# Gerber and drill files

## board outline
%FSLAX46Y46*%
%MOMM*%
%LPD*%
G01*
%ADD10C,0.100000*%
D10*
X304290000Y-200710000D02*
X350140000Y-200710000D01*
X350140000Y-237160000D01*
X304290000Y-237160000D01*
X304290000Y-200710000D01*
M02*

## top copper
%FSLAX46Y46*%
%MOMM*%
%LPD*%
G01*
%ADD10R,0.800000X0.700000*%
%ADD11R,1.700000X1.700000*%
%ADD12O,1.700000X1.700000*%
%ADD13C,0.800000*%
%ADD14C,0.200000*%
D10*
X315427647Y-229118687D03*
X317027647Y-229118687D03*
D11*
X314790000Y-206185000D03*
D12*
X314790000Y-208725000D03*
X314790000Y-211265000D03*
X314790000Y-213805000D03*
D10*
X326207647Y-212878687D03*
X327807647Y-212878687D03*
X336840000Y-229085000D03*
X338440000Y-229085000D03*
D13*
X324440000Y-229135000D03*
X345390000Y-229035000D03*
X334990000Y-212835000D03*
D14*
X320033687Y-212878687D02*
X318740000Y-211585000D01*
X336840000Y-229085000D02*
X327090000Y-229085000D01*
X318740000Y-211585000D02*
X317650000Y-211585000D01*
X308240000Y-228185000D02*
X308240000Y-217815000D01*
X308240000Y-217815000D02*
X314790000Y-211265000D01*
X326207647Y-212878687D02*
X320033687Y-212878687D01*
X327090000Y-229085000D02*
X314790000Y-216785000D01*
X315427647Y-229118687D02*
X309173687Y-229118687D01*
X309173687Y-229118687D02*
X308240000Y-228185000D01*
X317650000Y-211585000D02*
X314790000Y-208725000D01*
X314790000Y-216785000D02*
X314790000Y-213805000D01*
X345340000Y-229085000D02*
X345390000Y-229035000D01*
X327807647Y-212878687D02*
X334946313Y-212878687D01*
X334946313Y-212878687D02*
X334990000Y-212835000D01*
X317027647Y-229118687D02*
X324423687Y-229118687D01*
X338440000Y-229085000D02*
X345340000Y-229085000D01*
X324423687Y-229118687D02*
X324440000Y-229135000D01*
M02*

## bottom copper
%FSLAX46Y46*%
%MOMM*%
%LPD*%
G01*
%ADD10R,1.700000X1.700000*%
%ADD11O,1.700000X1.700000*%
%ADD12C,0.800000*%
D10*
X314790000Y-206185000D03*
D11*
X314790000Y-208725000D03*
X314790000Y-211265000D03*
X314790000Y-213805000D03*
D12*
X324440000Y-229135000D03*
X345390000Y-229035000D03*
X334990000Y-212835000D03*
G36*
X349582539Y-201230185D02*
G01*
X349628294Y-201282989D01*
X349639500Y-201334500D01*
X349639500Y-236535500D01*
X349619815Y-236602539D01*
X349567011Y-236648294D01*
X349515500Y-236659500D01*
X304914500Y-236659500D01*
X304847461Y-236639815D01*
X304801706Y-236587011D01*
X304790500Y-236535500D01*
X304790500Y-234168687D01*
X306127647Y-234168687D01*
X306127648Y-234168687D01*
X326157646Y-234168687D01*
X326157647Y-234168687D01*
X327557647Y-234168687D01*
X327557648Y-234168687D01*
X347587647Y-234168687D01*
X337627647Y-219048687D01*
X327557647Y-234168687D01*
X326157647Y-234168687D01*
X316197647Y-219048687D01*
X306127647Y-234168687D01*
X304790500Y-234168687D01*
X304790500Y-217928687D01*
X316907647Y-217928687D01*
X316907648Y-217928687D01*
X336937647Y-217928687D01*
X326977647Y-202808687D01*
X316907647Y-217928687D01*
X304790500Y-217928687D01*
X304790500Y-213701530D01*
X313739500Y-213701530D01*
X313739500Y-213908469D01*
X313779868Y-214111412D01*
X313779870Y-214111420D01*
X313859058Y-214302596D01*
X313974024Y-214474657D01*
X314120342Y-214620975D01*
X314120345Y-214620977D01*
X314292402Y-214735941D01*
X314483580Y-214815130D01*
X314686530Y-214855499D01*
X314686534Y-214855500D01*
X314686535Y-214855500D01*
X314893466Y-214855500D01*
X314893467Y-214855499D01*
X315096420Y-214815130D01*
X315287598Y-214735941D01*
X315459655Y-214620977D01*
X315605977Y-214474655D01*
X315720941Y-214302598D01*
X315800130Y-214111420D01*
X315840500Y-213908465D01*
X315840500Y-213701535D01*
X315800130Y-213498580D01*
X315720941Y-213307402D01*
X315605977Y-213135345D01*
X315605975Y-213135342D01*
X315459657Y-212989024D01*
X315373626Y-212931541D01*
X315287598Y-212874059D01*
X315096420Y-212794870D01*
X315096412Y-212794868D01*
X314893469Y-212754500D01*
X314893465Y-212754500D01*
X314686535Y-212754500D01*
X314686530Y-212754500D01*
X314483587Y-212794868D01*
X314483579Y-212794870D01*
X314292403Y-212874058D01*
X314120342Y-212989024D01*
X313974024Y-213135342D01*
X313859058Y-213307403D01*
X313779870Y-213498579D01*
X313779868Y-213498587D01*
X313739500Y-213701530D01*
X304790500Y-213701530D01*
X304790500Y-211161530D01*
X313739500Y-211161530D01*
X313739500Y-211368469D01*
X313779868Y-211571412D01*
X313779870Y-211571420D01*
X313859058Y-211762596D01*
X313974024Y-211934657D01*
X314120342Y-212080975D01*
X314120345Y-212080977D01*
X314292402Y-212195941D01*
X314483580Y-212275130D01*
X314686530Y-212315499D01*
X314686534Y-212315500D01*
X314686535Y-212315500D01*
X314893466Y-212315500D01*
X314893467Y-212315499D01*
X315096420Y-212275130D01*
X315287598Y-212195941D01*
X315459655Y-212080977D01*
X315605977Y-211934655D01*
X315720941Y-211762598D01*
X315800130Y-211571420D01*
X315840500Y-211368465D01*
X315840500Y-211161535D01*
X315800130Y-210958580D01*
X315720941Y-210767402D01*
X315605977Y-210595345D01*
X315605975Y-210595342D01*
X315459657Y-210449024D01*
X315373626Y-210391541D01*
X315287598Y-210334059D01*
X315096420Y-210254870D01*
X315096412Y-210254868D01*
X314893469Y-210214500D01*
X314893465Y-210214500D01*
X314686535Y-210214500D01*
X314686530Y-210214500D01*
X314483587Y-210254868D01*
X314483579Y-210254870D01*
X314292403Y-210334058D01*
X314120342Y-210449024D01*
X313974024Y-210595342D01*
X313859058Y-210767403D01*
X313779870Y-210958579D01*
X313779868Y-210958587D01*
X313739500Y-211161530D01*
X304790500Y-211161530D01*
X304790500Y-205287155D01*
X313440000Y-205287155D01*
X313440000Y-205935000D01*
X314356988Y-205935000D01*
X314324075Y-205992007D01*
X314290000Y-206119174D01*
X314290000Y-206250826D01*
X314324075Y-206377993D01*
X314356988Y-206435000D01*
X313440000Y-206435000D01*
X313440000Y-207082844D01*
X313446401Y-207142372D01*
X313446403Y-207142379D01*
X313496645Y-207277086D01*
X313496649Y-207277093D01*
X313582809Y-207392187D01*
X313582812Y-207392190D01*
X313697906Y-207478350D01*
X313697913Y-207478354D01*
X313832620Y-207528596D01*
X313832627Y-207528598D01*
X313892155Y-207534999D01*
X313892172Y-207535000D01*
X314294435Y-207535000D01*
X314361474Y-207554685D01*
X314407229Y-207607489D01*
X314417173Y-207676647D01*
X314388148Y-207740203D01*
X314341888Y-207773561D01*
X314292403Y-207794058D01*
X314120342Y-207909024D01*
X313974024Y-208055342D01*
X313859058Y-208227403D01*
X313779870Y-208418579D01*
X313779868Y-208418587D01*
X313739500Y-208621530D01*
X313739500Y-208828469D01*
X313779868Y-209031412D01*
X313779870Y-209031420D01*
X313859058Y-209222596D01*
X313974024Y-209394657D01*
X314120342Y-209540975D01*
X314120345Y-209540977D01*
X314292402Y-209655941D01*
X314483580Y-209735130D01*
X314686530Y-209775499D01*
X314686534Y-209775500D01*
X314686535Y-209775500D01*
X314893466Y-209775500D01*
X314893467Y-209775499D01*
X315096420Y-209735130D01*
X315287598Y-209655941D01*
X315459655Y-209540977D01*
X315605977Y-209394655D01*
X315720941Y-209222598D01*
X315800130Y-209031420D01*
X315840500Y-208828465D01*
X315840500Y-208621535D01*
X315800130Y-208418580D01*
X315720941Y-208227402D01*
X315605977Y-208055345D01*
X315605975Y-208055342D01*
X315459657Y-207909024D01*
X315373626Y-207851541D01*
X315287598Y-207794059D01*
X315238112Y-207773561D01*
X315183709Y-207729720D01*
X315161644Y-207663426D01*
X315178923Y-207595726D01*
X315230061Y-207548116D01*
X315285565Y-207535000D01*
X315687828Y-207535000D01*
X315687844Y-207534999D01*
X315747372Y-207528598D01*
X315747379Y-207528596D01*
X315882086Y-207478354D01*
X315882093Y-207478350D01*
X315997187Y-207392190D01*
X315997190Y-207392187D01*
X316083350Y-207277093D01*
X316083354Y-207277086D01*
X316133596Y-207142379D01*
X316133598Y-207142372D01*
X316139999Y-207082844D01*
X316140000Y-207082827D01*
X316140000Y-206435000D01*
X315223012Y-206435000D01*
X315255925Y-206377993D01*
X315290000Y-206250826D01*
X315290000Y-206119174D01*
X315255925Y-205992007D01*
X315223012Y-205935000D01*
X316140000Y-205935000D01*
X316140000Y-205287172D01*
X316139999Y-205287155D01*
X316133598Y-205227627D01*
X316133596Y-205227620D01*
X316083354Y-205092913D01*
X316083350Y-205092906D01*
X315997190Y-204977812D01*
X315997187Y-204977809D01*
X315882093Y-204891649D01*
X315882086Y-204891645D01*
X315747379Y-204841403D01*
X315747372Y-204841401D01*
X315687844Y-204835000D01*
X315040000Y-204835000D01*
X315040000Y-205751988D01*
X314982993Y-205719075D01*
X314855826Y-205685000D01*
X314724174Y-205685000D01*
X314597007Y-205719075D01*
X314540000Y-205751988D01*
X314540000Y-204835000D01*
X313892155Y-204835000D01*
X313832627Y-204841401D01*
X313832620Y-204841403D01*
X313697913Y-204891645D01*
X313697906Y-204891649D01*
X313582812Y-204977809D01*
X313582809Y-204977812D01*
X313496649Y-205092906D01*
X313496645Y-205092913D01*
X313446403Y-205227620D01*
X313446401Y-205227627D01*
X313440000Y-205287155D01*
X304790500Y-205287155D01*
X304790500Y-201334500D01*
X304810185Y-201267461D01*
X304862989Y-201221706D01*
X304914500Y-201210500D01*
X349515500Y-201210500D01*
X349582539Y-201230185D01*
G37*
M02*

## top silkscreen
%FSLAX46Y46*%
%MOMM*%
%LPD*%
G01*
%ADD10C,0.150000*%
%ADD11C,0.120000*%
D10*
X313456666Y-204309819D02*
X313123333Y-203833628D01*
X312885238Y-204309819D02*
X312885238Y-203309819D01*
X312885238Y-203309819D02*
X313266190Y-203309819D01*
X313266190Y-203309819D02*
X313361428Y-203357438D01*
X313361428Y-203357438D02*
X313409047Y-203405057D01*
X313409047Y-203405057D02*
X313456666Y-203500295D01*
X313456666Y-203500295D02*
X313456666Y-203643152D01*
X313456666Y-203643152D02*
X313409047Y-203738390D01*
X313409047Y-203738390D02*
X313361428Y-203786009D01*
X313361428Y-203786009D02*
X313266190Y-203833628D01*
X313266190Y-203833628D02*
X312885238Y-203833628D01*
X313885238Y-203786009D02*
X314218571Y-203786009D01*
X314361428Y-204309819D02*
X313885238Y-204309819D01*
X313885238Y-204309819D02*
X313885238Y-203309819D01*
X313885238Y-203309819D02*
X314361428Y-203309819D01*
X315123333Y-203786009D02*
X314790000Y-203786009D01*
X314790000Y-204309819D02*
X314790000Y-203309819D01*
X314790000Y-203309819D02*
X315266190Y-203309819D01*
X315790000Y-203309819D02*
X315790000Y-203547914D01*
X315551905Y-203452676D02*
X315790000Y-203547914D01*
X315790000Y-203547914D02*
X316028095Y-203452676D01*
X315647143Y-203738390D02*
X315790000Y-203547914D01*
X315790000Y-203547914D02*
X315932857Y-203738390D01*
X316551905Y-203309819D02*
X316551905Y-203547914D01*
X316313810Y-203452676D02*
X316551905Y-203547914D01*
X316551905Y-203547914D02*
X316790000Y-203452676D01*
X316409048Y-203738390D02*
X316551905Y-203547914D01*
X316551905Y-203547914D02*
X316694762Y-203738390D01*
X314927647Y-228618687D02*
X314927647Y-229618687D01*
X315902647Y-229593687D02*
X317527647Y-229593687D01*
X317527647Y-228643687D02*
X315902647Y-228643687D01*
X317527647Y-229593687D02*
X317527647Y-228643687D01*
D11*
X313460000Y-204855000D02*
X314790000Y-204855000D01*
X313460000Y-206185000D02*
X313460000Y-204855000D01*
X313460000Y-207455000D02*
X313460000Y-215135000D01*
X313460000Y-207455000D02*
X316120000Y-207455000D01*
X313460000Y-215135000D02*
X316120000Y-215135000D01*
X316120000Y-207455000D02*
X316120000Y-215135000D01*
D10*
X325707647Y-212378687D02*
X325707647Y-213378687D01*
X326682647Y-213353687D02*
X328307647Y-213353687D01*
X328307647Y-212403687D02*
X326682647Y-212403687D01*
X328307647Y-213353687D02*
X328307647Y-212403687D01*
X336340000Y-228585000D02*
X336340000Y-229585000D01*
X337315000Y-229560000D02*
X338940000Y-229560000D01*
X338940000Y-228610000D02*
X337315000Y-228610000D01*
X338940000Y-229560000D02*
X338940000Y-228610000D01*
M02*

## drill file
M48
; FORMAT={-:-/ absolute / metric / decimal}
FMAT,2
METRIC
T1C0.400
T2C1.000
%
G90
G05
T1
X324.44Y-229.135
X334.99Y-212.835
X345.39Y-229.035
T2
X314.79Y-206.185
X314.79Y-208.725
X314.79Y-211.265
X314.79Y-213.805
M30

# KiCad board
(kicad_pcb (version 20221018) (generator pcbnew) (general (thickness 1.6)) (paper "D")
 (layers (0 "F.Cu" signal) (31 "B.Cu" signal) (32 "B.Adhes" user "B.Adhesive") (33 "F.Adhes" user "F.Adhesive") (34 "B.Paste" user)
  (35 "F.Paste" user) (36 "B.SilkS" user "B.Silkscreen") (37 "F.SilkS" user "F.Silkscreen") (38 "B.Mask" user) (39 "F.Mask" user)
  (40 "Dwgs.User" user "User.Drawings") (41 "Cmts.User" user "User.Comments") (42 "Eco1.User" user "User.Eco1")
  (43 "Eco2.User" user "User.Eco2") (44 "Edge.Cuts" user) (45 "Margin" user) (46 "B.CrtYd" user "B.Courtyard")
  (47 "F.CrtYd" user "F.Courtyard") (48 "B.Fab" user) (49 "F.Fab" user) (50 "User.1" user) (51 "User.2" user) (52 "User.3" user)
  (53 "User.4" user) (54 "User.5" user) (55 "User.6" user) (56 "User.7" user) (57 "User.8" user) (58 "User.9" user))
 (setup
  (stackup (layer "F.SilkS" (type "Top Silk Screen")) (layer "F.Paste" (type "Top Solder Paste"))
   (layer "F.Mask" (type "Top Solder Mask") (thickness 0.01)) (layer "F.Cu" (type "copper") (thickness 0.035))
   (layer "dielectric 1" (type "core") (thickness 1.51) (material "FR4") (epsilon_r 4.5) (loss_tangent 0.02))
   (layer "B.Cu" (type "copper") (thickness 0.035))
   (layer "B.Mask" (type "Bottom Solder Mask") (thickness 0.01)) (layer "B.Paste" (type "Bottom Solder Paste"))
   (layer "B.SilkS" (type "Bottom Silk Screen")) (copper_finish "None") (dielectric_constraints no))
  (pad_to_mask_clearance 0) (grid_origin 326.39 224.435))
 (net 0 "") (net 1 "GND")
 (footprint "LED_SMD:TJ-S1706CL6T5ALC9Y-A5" (layer "F.Cu") (at 315.427647 229.118687)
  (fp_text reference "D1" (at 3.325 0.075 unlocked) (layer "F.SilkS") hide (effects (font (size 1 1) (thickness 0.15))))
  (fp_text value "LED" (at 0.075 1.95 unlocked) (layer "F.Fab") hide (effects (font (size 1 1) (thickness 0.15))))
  (fp_line (start -0.5 -0.5) (end -0.5 0.5) (stroke (width 0.15) (type default)) (layer "F.SilkS"))
  (fp_line (start 0.475 0.475) (end 2.1 0.475) (stroke (width 0.15) (type default)) (layer "F.SilkS"))
  (fp_line (start 2.1 -0.475) (end 0.475 -0.475) (stroke (width 0.15) (type default)) (layer "F.SilkS"))
  (fp_line (start 2.1 0.475) (end 2.1 -0.475) (stroke (width 0.15) (type default)) (layer "F.SilkS"))
  (pad "1" smd rect (at 0 0) (size 0.8 0.7) (layers "F.Cu" "F.Paste" "F.Mask") (thermal_bridge_angle 45))
  (pad "2" smd rect (at 1.6 0) (size 0.8 0.7) (layers "F.Cu" "F.Paste" "F.Mask") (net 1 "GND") (thermal_bridge_angle 45)))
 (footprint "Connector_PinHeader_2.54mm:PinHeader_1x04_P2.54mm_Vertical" (layer "F.Cu") (at 314.79 206.185)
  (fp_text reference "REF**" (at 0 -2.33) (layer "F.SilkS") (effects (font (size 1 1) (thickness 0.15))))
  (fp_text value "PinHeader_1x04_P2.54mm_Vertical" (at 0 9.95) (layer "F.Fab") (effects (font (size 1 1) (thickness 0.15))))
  (fp_line (start -1.33 -1.33) (end 0 -1.33) (stroke (width 0.12) (type solid)) (layer "F.SilkS"))
  (fp_line (start -1.33 0) (end -1.33 -1.33) (stroke (width 0.12) (type solid)) (layer "F.SilkS"))
  (fp_line (start -1.33 1.27) (end -1.33 8.95) (stroke (width 0.12) (type solid)) (layer "F.SilkS"))
  (fp_line (start -1.33 1.27) (end 1.33 1.27) (stroke (width 0.12) (type solid)) (layer "F.SilkS"))
  (fp_line (start -1.33 8.95) (end 1.33 8.95) (stroke (width 0.12) (type solid)) (layer "F.SilkS"))
  (fp_line (start 1.33 1.27) (end 1.33 8.95) (stroke (width 0.12) (type solid)) (layer "F.SilkS"))
  (pad "1" thru_hole rect (at 0 0) (size 1.7 1.7) (drill 1) (layers "*.Cu" "*.Mask") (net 1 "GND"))
  (pad "2" thru_hole oval (at 0 2.54) (size 1.7 1.7) (drill 1) (layers "*.Cu" "*.Mask"))
  (pad "3" thru_hole oval (at 0 5.08) (size 1.7 1.7) (drill 1) (layers "*.Cu" "*.Mask"))
  (pad "4" thru_hole oval (at 0 7.62) (size 1.7 1.7) (drill 1) (layers "*.Cu" "*.Mask")))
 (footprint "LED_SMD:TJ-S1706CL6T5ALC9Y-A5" (layer "F.Cu") (at 326.207647 212.878687)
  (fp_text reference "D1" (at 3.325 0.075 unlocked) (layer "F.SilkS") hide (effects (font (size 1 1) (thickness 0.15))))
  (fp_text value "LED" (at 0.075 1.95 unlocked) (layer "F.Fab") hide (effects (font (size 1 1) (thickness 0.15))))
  (fp_line (start -0.5 -0.5) (end -0.5 0.5) (stroke (width 0.15) (type default)) (layer "F.SilkS"))
  (fp_line (start 0.475 0.475) (end 2.1 0.475) (stroke (width 0.15) (type default)) (layer "F.SilkS"))
  (fp_line (start 2.1 -0.475) (end 0.475 -0.475) (stroke (width 0.15) (type default)) (layer "F.SilkS"))
  (fp_line (start 2.1 0.475) (end 2.1 -0.475) (stroke (width 0.15) (type default)) (layer "F.SilkS"))
  (pad "1" smd rect (at 0 0) (size 0.8 0.7) (layers "F.Cu" "F.Paste" "F.Mask") (thermal_bridge_angle 45))
  (pad "2" smd rect (at 1.6 0) (size 0.8 0.7) (layers "F.Cu" "F.Paste" "F.Mask") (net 1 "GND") (thermal_bridge_angle 45)))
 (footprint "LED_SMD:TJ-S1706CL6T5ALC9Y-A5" (layer "F.Cu") (at 336.84 229.085)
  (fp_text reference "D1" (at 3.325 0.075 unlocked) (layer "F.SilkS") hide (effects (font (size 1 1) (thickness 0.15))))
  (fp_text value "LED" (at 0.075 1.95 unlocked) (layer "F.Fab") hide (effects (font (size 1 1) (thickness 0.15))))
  (fp_line (start -0.5 -0.5) (end -0.5 0.5) (stroke (width 0.15) (type default)) (layer "F.SilkS"))
  (fp_line (start 0.475 0.475) (end 2.1 0.475) (stroke (width 0.15) (type default)) (layer "F.SilkS"))
  (fp_line (start 2.1 -0.475) (end 0.475 -0.475) (stroke (width 0.15) (type default)) (layer "F.SilkS"))
  (fp_line (start 2.1 0.475) (end 2.1 -0.475) (stroke (width 0.15) (type default)) (layer "F.SilkS"))
  (pad "1" smd rect (at 0 0) (size 0.8 0.7) (layers "F.Cu" "F.Paste" "F.Mask") (thermal_bridge_angle 45))
  (pad "2" smd rect (at 1.6 0) (size 0.8 0.7) (layers "F.Cu" "F.Paste" "F.Mask") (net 1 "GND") (thermal_bridge_angle 45)))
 (gr_rect (start 304.29 200.71) (end 350.14 237.16) (stroke (width 0.1) (type default)) (fill none) (layer "Edge.Cuts"))
 (segment (start 320.033687 212.878687) (end 318.74 211.585) (width 0.2) (layer "F.Cu") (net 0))
 (segment (start 336.84 229.085) (end 327.09 229.085) (width 0.2) (layer "F.Cu") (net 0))
 (segment (start 318.74 211.585) (end 317.65 211.585) (width 0.2) (layer "F.Cu") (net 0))
 (segment (start 308.24 228.185) (end 308.24 217.815) (width 0.2) (layer "F.Cu") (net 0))
 (segment (start 308.24 217.815) (end 314.79 211.265) (width 0.2) (layer "F.Cu") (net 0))
 (segment (start 326.207647 212.878687) (end 320.033687 212.878687) (width 0.2) (layer "F.Cu") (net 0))
 (segment (start 327.09 229.085) (end 314.79 216.785) (width 0.2) (layer "F.Cu") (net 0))
 (segment (start 315.427647 229.118687) (end 309.173687 229.118687) (width 0.2) (layer "F.Cu") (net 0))
 (segment (start 309.173687 229.118687) (end 308.24 228.185) (width 0.2) (layer "F.Cu") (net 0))
 (segment (start 317.65 211.585) (end 314.79 208.725) (width 0.2) (layer "F.Cu") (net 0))
 (segment (start 314.79 216.785) (end 314.79 213.805) (width 0.2) (layer "F.Cu") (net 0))
 (segment (start 345.34 229.085) (end 345.39 229.035) (width 0.2) (layer "F.Cu") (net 1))
 (segment (start 327.807647 212.878687) (end 334.946313 212.878687) (width 0.2) (layer "F.Cu") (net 1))
 (segment (start 334.946313 212.878687) (end 334.99 212.835) (width 0.2) (layer "F.Cu") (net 1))
 (segment (start 317.027647 229.118687) (end 324.423687 229.118687) (width 0.2) (layer "F.Cu") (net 1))
 (segment (start 338.44 229.085) (end 345.34 229.085) (width 0.2) (layer "F.Cu") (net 1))
 (segment (start 324.423687 229.118687) (end 324.44 229.135) (width 0.2) (layer "F.Cu") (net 1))
 (via (at 324.44 229.135) (size 0.8) (drill 0.4) (layers "F.Cu" "B.Cu") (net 1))
 (via (at 345.39 229.035) (size 0.8) (drill 0.4) (layers "F.Cu" "B.Cu") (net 1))
 (via (at 334.99 212.835) (size 0.8) (drill 0.4) (layers "F.Cu" "B.Cu") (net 1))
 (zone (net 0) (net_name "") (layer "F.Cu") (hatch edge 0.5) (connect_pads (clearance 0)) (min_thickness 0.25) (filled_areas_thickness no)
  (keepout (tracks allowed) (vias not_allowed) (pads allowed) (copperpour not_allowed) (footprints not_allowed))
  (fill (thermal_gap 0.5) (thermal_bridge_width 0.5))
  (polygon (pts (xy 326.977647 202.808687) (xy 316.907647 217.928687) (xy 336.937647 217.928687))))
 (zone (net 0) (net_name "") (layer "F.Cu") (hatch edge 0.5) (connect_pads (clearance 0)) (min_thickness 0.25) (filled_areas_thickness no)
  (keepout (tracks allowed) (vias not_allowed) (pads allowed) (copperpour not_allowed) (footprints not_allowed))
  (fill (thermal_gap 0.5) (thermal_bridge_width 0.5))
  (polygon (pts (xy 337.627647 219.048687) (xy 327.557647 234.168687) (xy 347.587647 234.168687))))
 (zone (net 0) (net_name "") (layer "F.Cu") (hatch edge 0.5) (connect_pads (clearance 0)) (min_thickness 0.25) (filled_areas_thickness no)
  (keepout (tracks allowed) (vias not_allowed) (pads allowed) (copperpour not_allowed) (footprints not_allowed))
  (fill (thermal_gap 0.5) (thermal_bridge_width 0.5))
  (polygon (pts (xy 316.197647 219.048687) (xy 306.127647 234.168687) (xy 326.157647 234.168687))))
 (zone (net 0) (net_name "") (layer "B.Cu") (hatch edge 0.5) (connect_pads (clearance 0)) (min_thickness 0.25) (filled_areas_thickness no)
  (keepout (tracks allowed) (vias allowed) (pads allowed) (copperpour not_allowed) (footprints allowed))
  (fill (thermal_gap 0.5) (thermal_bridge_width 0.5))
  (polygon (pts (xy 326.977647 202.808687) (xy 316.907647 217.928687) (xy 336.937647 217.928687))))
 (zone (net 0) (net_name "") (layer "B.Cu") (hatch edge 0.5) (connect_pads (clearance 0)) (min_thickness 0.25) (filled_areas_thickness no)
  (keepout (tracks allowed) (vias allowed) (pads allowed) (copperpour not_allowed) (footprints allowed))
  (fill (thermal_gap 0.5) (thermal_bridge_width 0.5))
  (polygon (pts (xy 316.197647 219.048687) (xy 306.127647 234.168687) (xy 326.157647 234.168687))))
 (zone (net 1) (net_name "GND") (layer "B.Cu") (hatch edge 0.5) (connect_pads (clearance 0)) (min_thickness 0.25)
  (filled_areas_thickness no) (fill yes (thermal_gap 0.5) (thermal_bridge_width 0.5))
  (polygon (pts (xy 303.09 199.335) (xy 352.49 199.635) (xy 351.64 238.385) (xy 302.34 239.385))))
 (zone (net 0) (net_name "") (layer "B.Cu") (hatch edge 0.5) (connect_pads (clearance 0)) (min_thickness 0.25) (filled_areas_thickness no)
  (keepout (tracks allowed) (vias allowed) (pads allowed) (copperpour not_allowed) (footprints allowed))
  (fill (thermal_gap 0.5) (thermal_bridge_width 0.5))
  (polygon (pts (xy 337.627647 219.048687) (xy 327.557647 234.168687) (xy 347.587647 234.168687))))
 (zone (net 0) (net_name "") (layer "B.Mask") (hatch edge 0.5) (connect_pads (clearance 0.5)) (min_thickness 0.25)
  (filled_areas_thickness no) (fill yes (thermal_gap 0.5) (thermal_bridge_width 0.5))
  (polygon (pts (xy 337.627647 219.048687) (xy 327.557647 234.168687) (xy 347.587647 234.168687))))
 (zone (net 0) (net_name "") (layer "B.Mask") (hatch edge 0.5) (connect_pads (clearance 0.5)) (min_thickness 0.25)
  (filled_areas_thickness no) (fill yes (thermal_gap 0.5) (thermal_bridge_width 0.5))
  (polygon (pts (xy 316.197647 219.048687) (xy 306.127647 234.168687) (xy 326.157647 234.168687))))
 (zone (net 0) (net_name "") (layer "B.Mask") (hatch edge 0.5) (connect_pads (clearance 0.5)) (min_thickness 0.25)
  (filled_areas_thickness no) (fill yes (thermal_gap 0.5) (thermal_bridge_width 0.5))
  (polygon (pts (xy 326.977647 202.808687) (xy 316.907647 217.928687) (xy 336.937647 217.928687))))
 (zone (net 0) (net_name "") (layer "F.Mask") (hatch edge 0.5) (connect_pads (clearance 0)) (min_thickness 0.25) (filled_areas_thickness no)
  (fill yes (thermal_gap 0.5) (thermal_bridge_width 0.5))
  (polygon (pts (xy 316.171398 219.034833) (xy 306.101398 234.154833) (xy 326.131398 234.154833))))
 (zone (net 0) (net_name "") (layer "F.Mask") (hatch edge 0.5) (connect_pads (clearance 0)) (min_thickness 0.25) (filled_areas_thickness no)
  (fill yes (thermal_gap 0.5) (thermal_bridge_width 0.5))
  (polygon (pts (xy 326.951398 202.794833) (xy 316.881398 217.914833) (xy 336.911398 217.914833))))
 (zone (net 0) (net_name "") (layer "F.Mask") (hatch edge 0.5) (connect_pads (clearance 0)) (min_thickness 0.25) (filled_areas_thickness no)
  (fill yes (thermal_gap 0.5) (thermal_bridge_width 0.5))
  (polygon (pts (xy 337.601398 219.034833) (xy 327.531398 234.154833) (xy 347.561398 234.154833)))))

